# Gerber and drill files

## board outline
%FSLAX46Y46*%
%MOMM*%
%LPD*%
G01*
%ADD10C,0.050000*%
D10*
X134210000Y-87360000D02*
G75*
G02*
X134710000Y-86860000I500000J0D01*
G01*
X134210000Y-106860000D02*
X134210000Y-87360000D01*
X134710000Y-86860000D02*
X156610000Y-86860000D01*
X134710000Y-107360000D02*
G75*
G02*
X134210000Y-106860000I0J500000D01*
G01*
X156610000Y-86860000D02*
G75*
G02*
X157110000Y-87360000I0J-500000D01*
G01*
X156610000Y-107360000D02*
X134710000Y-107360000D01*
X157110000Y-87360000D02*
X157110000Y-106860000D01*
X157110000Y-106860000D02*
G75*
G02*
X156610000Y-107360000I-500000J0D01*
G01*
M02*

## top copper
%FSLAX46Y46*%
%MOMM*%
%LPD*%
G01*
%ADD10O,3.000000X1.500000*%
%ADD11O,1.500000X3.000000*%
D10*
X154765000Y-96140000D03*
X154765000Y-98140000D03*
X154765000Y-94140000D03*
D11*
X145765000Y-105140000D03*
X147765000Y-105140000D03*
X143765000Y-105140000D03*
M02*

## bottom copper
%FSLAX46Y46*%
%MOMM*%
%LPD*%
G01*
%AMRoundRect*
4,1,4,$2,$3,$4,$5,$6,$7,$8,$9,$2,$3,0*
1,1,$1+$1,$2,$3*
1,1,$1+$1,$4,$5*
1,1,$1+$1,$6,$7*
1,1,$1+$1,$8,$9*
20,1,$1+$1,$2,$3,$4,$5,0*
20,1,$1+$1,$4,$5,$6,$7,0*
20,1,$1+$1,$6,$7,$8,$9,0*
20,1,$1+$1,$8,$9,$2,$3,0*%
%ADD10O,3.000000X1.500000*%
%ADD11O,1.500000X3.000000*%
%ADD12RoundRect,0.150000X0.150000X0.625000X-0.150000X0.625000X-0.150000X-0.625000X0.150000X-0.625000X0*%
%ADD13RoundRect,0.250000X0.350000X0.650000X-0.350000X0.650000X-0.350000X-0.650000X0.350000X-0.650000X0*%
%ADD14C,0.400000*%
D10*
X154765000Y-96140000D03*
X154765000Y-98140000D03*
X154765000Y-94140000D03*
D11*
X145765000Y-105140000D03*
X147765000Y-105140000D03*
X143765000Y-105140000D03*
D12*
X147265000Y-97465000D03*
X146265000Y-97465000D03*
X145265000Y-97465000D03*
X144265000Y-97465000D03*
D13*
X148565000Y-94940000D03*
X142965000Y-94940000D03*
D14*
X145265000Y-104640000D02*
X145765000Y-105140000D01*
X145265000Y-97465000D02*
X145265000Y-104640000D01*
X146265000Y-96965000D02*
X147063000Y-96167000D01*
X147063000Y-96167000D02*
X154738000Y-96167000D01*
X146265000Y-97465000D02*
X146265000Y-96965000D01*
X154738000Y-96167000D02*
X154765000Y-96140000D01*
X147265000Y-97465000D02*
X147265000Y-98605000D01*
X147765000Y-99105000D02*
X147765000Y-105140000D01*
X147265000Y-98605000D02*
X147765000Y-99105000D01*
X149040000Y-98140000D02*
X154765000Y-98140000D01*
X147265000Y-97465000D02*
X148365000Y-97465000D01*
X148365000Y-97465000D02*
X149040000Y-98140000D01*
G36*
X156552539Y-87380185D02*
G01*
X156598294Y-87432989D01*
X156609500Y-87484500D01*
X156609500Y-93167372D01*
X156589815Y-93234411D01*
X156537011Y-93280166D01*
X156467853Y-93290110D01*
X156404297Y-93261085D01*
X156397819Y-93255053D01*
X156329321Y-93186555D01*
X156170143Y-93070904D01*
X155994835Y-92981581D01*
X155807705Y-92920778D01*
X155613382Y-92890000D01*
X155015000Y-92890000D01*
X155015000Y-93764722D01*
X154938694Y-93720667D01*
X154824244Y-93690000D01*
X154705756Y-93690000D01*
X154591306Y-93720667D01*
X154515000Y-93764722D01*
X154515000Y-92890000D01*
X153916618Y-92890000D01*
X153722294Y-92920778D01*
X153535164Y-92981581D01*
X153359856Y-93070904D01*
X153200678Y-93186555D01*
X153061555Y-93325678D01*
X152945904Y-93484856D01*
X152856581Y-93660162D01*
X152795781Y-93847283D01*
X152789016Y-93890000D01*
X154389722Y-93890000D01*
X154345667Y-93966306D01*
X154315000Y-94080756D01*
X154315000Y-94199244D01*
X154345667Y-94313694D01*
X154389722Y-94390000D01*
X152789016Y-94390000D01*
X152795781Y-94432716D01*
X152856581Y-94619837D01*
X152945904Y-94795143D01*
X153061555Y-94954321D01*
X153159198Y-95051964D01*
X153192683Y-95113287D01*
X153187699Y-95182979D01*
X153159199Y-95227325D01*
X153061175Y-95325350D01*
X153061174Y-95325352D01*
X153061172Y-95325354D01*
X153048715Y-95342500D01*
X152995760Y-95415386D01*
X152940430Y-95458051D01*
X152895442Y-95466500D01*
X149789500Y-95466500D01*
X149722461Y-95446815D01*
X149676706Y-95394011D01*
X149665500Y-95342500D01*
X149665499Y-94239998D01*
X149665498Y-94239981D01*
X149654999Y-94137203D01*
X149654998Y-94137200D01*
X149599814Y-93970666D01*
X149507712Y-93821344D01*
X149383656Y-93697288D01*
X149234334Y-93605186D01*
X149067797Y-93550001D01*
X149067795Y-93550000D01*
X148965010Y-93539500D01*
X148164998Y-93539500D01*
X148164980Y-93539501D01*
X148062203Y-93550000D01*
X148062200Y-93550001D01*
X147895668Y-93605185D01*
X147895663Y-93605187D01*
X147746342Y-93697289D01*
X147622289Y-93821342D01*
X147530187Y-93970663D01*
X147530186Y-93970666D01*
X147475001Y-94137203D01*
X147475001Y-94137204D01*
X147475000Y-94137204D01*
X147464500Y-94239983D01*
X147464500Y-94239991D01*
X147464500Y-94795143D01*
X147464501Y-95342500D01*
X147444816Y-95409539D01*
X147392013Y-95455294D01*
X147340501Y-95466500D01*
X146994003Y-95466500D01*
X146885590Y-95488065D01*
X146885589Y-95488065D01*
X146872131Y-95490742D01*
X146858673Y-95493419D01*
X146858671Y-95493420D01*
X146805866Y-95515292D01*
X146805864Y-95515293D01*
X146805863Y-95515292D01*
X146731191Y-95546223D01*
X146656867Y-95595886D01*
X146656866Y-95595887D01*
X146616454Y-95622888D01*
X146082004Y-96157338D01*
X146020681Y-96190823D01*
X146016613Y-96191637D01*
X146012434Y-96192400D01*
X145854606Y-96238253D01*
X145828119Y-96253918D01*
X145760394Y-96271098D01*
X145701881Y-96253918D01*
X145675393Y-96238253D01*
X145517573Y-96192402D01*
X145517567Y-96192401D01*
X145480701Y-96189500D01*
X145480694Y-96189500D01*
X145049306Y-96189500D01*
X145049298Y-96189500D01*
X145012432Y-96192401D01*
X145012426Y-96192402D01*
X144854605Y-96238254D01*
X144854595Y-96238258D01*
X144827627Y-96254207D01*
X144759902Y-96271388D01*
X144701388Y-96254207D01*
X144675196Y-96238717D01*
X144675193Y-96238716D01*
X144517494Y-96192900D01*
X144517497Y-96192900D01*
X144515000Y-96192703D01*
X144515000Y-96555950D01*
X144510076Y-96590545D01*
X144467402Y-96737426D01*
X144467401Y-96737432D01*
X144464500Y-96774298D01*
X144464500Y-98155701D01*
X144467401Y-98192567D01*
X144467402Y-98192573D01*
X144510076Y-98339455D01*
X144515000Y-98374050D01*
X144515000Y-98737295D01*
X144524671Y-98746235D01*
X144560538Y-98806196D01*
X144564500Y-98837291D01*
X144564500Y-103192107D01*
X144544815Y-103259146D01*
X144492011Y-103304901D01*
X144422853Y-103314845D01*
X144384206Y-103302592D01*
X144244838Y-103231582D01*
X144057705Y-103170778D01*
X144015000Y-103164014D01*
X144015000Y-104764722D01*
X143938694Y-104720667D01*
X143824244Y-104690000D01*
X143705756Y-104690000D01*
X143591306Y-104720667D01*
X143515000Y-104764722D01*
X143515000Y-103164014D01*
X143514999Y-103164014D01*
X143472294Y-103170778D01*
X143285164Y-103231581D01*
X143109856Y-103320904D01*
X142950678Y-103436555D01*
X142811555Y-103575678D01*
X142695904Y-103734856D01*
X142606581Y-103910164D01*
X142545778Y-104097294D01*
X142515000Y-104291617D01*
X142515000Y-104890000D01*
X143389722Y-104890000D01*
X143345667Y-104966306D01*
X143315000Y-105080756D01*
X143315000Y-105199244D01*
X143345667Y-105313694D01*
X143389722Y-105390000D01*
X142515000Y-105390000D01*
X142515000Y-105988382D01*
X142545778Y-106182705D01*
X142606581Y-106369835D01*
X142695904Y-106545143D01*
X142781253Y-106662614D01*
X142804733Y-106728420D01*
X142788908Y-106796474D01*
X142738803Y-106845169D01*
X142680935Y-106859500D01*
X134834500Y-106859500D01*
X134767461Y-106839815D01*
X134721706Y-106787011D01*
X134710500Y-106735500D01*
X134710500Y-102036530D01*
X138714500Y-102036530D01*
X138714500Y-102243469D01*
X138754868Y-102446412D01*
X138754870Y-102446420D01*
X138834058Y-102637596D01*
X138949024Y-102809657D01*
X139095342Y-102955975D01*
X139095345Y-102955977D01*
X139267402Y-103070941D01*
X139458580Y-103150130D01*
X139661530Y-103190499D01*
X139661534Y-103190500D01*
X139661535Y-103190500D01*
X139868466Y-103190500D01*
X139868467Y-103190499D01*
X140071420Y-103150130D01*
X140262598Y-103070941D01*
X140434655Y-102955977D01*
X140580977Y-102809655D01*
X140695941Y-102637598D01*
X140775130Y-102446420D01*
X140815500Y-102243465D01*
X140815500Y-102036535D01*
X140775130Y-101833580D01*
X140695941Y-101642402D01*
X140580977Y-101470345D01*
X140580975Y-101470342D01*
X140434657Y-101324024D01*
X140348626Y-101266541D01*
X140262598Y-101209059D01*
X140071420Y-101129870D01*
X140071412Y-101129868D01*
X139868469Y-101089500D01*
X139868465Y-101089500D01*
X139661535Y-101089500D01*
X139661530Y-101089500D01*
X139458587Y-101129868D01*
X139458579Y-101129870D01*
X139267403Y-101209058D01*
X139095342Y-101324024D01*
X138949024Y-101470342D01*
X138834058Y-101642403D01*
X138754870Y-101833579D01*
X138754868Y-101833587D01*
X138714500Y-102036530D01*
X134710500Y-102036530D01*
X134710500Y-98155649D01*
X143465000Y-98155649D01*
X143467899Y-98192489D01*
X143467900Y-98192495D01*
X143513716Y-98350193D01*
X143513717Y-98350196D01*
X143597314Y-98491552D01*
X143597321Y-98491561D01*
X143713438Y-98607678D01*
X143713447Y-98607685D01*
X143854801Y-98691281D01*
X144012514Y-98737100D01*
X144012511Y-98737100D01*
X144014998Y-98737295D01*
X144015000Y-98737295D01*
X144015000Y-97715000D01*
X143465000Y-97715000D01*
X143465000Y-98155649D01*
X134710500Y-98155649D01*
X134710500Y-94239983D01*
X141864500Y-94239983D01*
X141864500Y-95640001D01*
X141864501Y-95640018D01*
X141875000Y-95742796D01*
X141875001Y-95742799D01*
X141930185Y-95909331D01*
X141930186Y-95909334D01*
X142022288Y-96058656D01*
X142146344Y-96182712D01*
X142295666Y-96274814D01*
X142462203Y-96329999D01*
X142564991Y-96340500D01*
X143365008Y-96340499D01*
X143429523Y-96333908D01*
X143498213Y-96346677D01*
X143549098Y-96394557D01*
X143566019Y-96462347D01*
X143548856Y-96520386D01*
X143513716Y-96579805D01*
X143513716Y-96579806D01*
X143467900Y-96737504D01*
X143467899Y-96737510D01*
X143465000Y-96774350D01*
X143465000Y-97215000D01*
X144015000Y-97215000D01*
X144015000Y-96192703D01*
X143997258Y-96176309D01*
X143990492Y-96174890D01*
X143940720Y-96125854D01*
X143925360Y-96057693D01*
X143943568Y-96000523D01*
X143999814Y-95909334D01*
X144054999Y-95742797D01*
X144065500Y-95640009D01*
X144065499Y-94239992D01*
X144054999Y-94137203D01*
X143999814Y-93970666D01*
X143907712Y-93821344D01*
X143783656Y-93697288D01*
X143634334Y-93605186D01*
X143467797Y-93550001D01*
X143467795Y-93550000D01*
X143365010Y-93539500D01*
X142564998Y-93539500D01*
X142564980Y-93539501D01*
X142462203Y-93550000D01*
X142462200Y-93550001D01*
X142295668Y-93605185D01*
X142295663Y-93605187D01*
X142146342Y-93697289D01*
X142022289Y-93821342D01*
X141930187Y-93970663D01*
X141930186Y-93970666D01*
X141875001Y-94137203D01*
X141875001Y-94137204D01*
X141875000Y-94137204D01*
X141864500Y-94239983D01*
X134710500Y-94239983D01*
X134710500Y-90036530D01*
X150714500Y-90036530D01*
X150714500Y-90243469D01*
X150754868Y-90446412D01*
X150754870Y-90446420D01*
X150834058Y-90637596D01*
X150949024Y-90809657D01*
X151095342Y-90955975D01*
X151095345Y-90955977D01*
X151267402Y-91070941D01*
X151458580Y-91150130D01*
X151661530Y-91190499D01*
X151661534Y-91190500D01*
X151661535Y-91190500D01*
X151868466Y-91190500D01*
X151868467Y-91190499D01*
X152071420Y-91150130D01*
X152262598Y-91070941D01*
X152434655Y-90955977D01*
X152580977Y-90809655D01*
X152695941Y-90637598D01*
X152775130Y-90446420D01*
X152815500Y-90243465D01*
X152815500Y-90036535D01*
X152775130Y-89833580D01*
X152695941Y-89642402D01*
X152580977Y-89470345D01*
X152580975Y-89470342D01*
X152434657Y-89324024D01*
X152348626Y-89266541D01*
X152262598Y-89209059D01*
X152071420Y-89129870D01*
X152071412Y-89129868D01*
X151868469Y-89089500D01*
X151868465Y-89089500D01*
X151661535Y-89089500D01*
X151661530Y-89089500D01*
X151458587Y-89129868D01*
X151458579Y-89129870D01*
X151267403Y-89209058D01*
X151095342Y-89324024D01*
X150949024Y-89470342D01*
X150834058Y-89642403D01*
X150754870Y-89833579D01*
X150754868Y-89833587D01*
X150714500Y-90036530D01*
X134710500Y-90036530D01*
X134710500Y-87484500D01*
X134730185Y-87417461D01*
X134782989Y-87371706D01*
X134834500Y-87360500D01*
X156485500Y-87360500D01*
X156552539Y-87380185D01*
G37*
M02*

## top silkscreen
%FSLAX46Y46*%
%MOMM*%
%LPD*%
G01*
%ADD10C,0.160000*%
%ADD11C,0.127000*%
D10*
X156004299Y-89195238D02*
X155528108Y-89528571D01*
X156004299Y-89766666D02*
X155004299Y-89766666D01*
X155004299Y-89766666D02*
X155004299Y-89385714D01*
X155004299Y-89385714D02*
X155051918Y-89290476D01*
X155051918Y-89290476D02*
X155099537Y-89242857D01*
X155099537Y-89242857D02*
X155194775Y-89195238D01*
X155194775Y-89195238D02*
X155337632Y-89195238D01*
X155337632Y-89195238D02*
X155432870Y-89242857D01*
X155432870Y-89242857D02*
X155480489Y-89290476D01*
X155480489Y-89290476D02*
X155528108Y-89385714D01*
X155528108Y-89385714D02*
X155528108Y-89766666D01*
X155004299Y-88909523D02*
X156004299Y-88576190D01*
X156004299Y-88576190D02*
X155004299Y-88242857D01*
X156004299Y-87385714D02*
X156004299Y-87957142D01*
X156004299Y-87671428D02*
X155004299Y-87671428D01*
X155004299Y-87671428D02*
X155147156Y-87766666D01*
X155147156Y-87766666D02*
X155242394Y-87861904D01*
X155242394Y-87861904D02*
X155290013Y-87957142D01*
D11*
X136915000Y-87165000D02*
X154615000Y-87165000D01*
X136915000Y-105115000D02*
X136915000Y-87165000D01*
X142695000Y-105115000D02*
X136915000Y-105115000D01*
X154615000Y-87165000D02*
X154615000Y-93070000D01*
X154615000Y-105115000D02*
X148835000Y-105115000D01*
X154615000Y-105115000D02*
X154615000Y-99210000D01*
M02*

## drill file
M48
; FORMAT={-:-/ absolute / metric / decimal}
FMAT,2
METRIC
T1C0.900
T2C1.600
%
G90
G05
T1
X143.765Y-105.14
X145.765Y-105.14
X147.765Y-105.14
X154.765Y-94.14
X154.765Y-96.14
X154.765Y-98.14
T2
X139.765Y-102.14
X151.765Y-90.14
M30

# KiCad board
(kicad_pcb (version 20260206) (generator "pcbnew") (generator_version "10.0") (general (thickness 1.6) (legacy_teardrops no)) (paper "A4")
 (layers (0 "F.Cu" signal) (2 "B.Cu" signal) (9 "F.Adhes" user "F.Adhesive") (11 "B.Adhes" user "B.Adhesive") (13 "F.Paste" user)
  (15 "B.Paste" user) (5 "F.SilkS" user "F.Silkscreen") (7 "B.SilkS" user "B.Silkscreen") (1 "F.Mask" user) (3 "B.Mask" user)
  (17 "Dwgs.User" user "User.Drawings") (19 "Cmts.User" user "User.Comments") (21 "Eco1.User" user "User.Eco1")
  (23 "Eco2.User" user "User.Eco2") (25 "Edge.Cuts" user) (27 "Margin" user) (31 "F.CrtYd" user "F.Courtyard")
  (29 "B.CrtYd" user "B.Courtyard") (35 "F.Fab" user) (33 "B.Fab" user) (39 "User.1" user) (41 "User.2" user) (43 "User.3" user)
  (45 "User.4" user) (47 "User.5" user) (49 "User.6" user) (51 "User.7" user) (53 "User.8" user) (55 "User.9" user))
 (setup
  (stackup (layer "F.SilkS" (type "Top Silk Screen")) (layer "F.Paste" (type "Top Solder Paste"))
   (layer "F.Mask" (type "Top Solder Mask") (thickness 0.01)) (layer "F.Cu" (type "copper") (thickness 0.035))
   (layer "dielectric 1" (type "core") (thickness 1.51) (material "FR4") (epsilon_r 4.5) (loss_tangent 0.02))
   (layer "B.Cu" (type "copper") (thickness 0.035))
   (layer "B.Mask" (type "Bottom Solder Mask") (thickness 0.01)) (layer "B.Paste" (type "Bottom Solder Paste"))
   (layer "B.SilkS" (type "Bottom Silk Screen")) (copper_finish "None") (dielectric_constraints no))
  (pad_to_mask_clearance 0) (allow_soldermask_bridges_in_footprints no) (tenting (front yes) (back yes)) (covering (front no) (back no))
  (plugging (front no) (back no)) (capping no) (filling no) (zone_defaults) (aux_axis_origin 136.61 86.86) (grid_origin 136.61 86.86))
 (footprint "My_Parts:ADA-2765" (layer "F.Cu") (at 145.765 96.14)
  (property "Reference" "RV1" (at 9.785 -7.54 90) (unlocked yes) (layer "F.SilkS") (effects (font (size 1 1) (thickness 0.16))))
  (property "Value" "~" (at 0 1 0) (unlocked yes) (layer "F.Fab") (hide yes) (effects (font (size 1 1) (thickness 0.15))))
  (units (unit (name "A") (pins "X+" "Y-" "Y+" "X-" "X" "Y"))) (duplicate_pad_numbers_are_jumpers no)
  (fp_line (start -8.85 -8.975) (end 8.85 -8.975) (stroke (width 0.127) (type solid)) (layer "F.SilkS"))
  (fp_line (start -8.85 8.975) (end -8.85 -8.975) (stroke (width 0.127) (type solid)) (layer "F.SilkS"))
  (fp_line (start -3.07 8.975) (end -8.85 8.975) (stroke (width 0.127) (type solid)) (layer "F.SilkS"))
  (fp_line (start 8.85 -8.975) (end 8.85 -3.07) (stroke (width 0.127) (type solid)) (layer "F.SilkS"))
  (fp_line (start 8.85 8.975) (end 3.07 8.975) (stroke (width 0.127) (type solid)) (layer "F.SilkS"))
  (fp_line (start 8.85 8.975) (end 8.85 3.07) (stroke (width 0.127) (type solid)) (layer "F.SilkS"))
  (pad "" np_thru_hole circle (at -6 6) (size 1.6 1.6) (drill 1.6) (layers "*.Cu" "*.Mask"))
  (pad "" np_thru_hole circle (at 6 -6) (size 1.6 1.6) (drill 1.6) (layers "*.Cu" "*.Mask"))
  (pad "X" thru_hole oval (at 9 0) (size 3 1.5) (drill 0.9) (layers "*.Cu" "*.Mask") (remove_unused_layers no) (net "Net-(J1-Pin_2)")
   (solder_mask_margin 0.102))
  (pad "X+" thru_hole oval (at 9 2) (size 3 1.5) (drill 0.9) (layers "*.Cu" "*.Mask") (remove_unused_layers no) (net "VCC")
   (solder_mask_margin 0.102))
  (pad "X-" thru_hole oval (at 9 -2) (size 3 1.5) (drill 0.9) (layers "*.Cu" "*.Mask") (remove_unused_layers no) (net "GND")
   (solder_mask_margin 0.102))
  (pad "Y" thru_hole oval (at 0 9) (size 1.5 3) (drill 0.9) (layers "*.Cu" "*.Mask") (remove_unused_layers no) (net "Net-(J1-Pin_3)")
   (solder_mask_margin 0.102))
  (pad "Y+" thru_hole oval (at 2 9) (size 1.5 3) (drill 0.9) (layers "*.Cu" "*.Mask") (remove_unused_layers no) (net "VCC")
   (solder_mask_margin 0.102))
  (pad "Y-" thru_hole oval (at -2 9) (size 1.5 3) (drill 0.9) (layers "*.Cu" "*.Mask") (remove_unused_layers no) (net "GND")
   (solder_mask_margin 0.102)))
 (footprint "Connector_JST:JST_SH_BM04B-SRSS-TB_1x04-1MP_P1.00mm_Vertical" (layer "B.Cu") (at 145.765 96.14 180)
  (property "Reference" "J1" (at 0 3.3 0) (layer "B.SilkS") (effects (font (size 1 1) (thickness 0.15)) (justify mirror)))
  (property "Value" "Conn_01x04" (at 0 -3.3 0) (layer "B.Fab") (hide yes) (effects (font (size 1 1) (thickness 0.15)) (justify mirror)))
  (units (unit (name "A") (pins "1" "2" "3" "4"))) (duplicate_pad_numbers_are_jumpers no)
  (pad "1" smd roundrect (at -1.5 -1.325 180) (size 0.6 1.55) (layers "B.Cu" "B.Mask" "B.Paste") (roundrect_rratio 0.25) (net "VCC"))
  (pad "2" smd roundrect (at -0.5 -1.325 180) (size 0.6 1.55) (layers "B.Cu" "B.Mask" "B.Paste") (roundrect_rratio 0.25)
   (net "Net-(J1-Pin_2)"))
  (pad "3" smd roundrect (at 0.5 -1.325 180) (size 0.6 1.55) (layers "B.Cu" "B.Mask" "B.Paste") (roundrect_rratio 0.25)
   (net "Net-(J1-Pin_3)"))
  (pad "4" smd roundrect (at 1.5 -1.325 180) (size 0.6 1.55) (layers "B.Cu" "B.Mask" "B.Paste") (roundrect_rratio 0.25) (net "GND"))
  (pad "MP" smd roundrect (at -2.8 1.2 180) (size 1.2 1.8) (layers "B.Cu" "B.Mask" "B.Paste") (roundrect_rratio 0.208333))
  (pad "MP" smd roundrect (at 2.8 1.2 180) (size 1.2 1.8) (layers "B.Cu" "B.Mask" "B.Paste") (roundrect_rratio 0.208333)))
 (gr_arc (start 134.21 87.36) (mid 134.356447 87.006447) (end 134.71 86.86) (stroke (width 0.05) (type solid)) (layer "Edge.Cuts"))
 (gr_line (start 134.21 106.86) (end 134.21 87.36) (stroke (width 0.05) (type solid)) (layer "Edge.Cuts"))
 (gr_line (start 134.71 86.86) (end 156.61 86.86) (stroke (width 0.05) (type default)) (layer "Edge.Cuts"))
 (gr_arc (start 134.71 107.36) (mid 134.356447 107.213553) (end 134.21 106.86) (stroke (width 0.05) (type default)) (layer "Edge.Cuts"))
 (gr_arc (start 156.61 86.86) (mid 156.963553 87.006447) (end 157.11 87.36) (stroke (width 0.05) (type default)) (layer "Edge.Cuts"))
 (gr_line (start 156.61 107.36) (end 134.71 107.36) (stroke (width 0.05) (type default)) (layer "Edge.Cuts"))
 (gr_line (start 157.11 87.36) (end 157.11 106.86) (stroke (width 0.05) (type default)) (layer "Edge.Cuts"))
 (gr_arc (start 157.11 106.86) (mid 156.963553 107.213553) (end 156.61 107.36) (stroke (width 0.05) (type default)) (layer "Edge.Cuts"))
 (segment (start 145.265 104.64) (end 145.765 105.14) (width 0.4) (layer "B.Cu") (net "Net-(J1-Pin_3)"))
 (segment (start 145.265 97.465) (end 145.265 104.64) (width 0.4) (layer "B.Cu") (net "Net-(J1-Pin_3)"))
 (segment (start 146.265 96.965) (end 147.063 96.167) (width 0.4) (layer "B.Cu") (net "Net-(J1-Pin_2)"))
 (segment (start 147.063 96.167) (end 154.738 96.167) (width 0.4) (layer "B.Cu") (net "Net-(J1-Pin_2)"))
 (segment (start 146.265 97.465) (end 146.265 96.965) (width 0.4) (layer "B.Cu") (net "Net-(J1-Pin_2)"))
 (segment (start 154.738 96.167) (end 154.765 96.14) (width 0.4) (layer "B.Cu") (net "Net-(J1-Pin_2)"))
 (segment (start 147.265 97.465) (end 147.265 98.605) (width 0.4) (layer "B.Cu") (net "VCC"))
 (segment (start 147.765 99.105) (end 147.765 105.14) (width 0.4) (layer "B.Cu") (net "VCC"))
 (segment (start 147.265 98.605) (end 147.765 99.105) (width 0.4) (layer "B.Cu") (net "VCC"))
 (segment (start 149.04 98.14) (end 154.765 98.14) (width 0.4) (layer "B.Cu") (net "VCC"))
 (segment (start 147.265 97.465) (end 148.365 97.465) (width 0.4) (layer "B.Cu") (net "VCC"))
 (segment (start 148.365 97.465) (end 149.04 98.14) (width 0.4) (layer "B.Cu") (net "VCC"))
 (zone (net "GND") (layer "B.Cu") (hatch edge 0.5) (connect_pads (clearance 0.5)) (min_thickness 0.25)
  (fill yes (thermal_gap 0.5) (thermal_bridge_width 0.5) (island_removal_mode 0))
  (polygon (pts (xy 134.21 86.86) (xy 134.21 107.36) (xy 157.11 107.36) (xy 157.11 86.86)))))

